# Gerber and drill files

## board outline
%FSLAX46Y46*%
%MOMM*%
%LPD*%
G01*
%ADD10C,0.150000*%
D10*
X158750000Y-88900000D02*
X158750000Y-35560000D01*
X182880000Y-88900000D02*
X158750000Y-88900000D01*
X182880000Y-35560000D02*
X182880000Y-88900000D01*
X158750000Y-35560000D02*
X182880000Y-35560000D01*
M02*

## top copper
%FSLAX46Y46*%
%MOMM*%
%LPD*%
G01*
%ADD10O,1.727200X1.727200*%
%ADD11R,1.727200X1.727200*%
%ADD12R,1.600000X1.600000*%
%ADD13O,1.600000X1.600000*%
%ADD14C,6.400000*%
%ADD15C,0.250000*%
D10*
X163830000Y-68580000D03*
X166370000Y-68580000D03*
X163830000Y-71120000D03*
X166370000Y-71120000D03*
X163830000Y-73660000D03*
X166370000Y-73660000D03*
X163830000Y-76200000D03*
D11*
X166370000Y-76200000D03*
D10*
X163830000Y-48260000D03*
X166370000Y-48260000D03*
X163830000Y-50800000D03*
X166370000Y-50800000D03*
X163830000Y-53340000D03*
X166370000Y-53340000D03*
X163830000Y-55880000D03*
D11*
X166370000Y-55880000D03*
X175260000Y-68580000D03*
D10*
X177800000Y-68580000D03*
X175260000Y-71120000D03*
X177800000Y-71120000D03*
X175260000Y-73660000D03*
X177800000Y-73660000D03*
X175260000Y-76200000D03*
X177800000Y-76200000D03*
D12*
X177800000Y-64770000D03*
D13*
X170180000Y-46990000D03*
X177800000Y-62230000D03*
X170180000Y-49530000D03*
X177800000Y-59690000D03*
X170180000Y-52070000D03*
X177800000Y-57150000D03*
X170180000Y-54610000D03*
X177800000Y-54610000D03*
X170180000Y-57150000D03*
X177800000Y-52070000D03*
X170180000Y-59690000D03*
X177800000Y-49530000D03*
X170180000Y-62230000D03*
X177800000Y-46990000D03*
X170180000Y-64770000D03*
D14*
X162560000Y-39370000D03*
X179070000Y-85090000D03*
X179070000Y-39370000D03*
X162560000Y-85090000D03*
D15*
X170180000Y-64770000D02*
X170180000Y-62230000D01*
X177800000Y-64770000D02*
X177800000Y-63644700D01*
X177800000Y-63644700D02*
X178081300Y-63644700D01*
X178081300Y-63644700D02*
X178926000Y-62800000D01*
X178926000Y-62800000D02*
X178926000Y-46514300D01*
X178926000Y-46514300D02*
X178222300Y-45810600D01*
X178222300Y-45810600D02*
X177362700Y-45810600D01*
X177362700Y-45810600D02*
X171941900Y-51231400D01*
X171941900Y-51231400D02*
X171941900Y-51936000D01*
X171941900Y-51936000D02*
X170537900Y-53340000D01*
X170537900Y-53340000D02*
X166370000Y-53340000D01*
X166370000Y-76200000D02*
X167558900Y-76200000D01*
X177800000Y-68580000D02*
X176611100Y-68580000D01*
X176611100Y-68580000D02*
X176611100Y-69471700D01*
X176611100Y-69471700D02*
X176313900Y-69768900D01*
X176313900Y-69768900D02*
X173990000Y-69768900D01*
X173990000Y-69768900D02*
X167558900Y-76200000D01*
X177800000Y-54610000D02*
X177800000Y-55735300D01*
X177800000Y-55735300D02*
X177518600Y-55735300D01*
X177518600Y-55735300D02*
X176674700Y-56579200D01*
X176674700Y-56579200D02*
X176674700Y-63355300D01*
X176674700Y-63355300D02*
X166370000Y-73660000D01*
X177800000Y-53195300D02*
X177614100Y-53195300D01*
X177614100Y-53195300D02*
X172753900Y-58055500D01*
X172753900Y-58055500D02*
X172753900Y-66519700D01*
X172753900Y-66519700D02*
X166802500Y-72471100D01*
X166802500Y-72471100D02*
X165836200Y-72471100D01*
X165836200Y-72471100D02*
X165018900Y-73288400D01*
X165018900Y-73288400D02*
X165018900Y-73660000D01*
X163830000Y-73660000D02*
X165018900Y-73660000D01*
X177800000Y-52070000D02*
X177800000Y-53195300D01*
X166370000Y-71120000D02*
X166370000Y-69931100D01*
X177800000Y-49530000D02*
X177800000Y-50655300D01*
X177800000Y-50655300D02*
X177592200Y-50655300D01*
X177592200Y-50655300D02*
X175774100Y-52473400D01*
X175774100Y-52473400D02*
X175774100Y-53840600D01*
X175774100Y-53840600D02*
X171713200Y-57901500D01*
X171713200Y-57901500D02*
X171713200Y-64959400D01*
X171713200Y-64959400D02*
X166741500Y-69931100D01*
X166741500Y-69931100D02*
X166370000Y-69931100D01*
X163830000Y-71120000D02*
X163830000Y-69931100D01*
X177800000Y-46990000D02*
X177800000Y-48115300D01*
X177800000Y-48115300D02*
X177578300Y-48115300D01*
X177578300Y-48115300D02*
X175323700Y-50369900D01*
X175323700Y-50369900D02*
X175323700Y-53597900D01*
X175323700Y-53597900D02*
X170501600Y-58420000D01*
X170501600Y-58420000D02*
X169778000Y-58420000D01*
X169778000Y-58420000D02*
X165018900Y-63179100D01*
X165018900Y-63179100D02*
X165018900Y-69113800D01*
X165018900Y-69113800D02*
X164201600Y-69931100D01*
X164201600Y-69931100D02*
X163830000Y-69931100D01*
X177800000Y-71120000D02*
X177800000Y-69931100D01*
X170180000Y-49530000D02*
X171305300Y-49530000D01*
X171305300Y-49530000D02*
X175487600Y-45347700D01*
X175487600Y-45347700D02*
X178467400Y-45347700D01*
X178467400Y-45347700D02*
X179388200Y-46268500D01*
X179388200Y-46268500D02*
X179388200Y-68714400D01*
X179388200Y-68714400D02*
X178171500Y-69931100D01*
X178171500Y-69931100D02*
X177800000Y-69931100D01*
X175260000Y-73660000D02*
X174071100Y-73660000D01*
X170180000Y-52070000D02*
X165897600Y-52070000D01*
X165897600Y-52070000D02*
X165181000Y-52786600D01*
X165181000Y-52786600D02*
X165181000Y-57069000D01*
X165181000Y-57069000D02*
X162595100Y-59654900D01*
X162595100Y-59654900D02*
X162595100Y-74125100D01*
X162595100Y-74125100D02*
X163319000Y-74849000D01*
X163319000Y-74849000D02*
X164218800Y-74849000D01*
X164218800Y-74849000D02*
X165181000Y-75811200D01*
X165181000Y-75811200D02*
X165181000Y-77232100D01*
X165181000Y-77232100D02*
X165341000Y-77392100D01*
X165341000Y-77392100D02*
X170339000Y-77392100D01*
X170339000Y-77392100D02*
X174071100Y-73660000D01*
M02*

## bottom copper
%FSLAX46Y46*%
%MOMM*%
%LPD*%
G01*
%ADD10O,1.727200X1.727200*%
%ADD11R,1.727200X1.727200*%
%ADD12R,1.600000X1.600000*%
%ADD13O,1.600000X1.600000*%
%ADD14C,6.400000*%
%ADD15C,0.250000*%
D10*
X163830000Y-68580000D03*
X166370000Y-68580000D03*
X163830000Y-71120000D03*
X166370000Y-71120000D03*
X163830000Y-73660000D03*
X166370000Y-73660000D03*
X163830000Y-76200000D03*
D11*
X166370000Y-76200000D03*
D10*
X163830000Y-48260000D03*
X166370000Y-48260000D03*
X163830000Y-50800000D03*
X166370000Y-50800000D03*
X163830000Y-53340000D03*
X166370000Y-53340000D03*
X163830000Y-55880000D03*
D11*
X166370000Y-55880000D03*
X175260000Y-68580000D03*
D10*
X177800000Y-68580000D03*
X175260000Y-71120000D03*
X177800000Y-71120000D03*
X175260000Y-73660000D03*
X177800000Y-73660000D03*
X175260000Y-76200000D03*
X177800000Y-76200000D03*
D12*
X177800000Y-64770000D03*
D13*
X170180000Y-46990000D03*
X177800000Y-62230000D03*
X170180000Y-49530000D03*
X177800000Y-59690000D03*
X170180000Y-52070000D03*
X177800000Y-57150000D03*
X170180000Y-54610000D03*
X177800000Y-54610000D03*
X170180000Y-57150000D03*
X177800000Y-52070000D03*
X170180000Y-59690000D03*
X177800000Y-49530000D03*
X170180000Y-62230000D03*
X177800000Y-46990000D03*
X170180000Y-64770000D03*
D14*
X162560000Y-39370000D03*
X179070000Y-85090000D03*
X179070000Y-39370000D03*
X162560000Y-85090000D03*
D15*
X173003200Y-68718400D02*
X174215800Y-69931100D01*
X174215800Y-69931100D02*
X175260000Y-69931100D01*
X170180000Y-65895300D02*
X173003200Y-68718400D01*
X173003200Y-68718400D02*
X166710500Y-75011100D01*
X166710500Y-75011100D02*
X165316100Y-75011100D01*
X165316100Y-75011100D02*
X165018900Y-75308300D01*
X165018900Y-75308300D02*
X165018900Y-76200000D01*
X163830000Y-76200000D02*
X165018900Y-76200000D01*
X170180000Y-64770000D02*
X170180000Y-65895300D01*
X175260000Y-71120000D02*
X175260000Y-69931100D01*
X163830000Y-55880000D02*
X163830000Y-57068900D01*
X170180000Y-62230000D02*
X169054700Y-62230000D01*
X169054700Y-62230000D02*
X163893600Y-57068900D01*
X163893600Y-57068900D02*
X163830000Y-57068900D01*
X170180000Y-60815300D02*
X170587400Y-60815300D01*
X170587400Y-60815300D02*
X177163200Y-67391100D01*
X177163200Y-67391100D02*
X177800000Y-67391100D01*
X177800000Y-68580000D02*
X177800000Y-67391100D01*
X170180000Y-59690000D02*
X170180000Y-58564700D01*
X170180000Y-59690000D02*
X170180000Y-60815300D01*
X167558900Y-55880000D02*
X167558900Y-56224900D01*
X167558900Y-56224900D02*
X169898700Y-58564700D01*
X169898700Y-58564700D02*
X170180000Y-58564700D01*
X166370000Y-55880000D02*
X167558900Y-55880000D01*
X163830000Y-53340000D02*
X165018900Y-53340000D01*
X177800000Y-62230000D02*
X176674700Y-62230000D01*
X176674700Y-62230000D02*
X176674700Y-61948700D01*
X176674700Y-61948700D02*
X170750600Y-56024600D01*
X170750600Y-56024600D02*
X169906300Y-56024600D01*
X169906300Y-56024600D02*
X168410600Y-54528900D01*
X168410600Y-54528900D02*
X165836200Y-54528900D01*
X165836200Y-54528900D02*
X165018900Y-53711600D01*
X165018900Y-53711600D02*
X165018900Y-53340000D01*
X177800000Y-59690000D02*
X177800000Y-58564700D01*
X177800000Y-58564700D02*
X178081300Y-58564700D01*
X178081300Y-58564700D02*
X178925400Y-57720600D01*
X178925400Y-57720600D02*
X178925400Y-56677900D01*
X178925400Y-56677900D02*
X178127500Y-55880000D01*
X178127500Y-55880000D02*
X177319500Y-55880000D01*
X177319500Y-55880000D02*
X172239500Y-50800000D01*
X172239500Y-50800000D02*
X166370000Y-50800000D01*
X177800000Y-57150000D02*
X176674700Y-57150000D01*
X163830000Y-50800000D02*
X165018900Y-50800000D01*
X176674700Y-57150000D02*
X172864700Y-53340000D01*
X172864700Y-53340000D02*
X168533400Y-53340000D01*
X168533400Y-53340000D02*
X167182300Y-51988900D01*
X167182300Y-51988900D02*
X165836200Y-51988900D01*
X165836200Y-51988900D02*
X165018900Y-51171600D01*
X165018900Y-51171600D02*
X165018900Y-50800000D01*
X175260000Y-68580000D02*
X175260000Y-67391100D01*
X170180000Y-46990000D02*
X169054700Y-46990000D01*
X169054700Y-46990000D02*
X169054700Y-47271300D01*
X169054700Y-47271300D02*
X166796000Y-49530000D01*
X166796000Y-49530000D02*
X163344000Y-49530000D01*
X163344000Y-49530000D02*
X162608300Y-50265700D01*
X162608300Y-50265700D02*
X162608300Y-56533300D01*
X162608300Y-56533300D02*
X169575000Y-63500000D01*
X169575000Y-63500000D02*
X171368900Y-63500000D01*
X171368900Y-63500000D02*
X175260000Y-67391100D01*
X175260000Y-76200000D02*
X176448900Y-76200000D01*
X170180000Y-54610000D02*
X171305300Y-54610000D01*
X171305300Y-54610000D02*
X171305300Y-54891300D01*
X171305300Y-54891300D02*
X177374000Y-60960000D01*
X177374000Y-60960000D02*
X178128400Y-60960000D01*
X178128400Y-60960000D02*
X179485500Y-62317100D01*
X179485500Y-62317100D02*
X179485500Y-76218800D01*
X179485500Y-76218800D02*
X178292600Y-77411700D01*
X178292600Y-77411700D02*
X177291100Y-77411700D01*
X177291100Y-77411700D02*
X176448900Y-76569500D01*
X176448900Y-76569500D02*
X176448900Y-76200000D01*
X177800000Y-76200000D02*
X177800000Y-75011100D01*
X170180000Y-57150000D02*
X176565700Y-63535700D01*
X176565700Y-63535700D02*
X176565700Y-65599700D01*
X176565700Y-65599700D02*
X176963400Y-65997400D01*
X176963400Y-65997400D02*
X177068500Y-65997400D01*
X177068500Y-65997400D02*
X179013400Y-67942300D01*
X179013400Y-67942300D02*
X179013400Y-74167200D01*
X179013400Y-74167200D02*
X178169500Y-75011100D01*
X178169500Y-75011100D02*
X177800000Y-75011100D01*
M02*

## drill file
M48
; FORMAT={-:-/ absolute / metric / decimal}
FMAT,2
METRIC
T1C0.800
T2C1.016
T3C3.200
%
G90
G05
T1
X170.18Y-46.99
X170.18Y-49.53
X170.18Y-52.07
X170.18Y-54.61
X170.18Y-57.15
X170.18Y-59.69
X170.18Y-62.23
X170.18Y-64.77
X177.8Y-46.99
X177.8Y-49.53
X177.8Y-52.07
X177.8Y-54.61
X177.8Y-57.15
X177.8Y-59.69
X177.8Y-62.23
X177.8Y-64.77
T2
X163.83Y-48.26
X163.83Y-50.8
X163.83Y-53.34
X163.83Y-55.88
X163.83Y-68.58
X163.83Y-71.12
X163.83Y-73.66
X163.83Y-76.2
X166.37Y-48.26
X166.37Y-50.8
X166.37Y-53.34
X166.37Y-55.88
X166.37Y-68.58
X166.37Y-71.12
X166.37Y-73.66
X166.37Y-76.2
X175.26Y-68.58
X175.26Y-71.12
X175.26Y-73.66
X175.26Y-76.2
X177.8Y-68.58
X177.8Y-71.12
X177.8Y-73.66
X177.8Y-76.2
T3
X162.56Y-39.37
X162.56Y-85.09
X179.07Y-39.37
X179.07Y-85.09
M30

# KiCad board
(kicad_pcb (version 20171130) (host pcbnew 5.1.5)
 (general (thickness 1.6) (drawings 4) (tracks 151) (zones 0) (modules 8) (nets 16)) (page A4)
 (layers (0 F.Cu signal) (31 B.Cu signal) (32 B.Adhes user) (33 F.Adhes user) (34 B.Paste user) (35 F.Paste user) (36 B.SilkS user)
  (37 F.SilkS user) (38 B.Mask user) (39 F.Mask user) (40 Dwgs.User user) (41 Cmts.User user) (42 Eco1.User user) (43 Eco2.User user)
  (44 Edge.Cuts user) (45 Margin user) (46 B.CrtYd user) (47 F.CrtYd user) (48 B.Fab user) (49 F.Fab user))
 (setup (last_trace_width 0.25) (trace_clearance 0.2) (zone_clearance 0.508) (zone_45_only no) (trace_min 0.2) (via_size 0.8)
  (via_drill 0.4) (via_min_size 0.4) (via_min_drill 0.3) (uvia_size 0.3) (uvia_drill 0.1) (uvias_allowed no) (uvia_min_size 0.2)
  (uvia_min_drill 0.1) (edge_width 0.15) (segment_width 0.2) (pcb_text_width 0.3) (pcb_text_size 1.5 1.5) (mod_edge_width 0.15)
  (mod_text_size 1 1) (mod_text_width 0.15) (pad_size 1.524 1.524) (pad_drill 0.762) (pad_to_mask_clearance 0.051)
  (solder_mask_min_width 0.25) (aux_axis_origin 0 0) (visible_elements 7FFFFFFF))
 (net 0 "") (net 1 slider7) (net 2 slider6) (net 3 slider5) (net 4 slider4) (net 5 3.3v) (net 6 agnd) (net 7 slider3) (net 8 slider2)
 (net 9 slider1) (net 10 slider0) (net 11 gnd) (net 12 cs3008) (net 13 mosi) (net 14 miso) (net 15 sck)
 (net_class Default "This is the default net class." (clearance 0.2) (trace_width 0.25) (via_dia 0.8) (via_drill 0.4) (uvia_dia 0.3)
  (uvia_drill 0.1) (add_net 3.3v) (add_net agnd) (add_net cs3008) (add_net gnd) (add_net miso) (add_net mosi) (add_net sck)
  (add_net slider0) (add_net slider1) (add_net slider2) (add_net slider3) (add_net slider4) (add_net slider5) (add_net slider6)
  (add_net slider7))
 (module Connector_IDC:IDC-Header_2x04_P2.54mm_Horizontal (layer F.Cu) (at 166.37 76.2 180)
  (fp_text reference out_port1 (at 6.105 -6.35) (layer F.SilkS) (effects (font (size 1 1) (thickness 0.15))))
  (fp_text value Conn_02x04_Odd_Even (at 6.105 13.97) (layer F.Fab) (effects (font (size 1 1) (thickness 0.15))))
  (pad 8 thru_hole oval (at 2.54 7.62 180) (size 1.7272 1.7272) (drill 1.016) (layers *.Cu *.Mask))
  (pad 7 thru_hole oval (at 0 7.62 180) (size 1.7272 1.7272) (drill 1.016) (layers *.Cu *.Mask))
  (pad 6 thru_hole oval (at 2.54 5.08 180) (size 1.7272 1.7272) (drill 1.016) (layers *.Cu *.Mask) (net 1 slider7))
  (pad 5 thru_hole oval (at 0 5.08 180) (size 1.7272 1.7272) (drill 1.016) (layers *.Cu *.Mask) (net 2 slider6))
  (pad 4 thru_hole oval (at 2.54 2.54 180) (size 1.7272 1.7272) (drill 1.016) (layers *.Cu *.Mask) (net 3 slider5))
  (pad 3 thru_hole oval (at 0 2.54 180) (size 1.7272 1.7272) (drill 1.016) (layers *.Cu *.Mask) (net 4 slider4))
  (pad 2 thru_hole oval (at 2.54 0 180) (size 1.7272 1.7272) (drill 1.016) (layers *.Cu *.Mask) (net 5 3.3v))
  (pad 1 thru_hole rect (at 0 0 180) (size 1.7272 1.7272) (drill 1.016) (layers *.Cu *.Mask) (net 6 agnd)))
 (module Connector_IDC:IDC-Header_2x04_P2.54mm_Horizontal (layer F.Cu) (at 166.37 55.88 180)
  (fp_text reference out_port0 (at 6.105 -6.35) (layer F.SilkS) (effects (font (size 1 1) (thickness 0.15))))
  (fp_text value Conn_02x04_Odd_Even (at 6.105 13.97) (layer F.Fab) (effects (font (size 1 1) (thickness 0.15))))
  (pad 8 thru_hole oval (at 2.54 7.62 180) (size 1.7272 1.7272) (drill 1.016) (layers *.Cu *.Mask))
  (pad 7 thru_hole oval (at 0 7.62 180) (size 1.7272 1.7272) (drill 1.016) (layers *.Cu *.Mask))
  (pad 6 thru_hole oval (at 2.54 5.08 180) (size 1.7272 1.7272) (drill 1.016) (layers *.Cu *.Mask) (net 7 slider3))
  (pad 5 thru_hole oval (at 0 5.08 180) (size 1.7272 1.7272) (drill 1.016) (layers *.Cu *.Mask) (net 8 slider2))
  (pad 4 thru_hole oval (at 2.54 2.54 180) (size 1.7272 1.7272) (drill 1.016) (layers *.Cu *.Mask) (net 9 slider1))
  (pad 3 thru_hole oval (at 0 2.54 180) (size 1.7272 1.7272) (drill 1.016) (layers *.Cu *.Mask) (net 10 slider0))
  (pad 2 thru_hole oval (at 2.54 0 180) (size 1.7272 1.7272) (drill 1.016) (layers *.Cu *.Mask) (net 5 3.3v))
  (pad 1 thru_hole rect (at 0 0 180) (size 1.7272 1.7272) (drill 1.016) (layers *.Cu *.Mask) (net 6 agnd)))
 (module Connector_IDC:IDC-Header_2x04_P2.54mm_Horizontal (layer F.Cu) (at 175.26 68.58)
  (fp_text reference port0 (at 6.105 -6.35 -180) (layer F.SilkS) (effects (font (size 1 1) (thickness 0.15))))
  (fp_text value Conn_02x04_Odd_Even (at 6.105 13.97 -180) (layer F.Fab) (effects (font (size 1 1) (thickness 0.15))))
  (pad 1 thru_hole rect (at 0 0) (size 1.7272 1.7272) (drill 1.016) (layers *.Cu *.Mask) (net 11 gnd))
  (pad 2 thru_hole oval (at 2.54 0) (size 1.7272 1.7272) (drill 1.016) (layers *.Cu *.Mask) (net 6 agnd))
  (pad 3 thru_hole oval (at 0 2.54) (size 1.7272 1.7272) (drill 1.016) (layers *.Cu *.Mask) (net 5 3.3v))
  (pad 4 thru_hole oval (at 2.54 2.54) (size 1.7272 1.7272) (drill 1.016) (layers *.Cu *.Mask) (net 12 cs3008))
  (pad 5 thru_hole oval (at 0 5.08) (size 1.7272 1.7272) (drill 1.016) (layers *.Cu *.Mask) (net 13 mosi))
  (pad 6 thru_hole oval (at 2.54 5.08) (size 1.7272 1.7272) (drill 1.016) (layers *.Cu *.Mask))
  (pad 7 thru_hole oval (at 0 7.62) (size 1.7272 1.7272) (drill 1.016) (layers *.Cu *.Mask) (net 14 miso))
  (pad 8 thru_hole oval (at 2.54 7.62) (size 1.7272 1.7272) (drill 1.016) (layers *.Cu *.Mask) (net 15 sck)))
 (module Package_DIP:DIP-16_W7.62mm (layer F.Cu) (at 177.8 64.77 180)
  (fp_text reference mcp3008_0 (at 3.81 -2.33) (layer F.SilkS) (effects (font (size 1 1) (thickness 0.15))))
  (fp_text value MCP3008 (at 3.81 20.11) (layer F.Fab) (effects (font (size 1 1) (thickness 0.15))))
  (pad 1 thru_hole rect (at 0 0 180) (size 1.6 1.6) (drill 0.8) (layers *.Cu *.Mask) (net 10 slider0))
  (pad 9 thru_hole oval (at 7.62 17.78 180) (size 1.6 1.6) (drill 0.8) (layers *.Cu *.Mask) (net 11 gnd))
  (pad 2 thru_hole oval (at 0 2.54 180) (size 1.6 1.6) (drill 0.8) (layers *.Cu *.Mask) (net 9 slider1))
  (pad 10 thru_hole oval (at 7.62 15.24 180) (size 1.6 1.6) (drill 0.8) (layers *.Cu *.Mask) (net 12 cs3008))
  (pad 3 thru_hole oval (at 0 5.08 180) (size 1.6 1.6) (drill 0.8) (layers *.Cu *.Mask) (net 8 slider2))
  (pad 11 thru_hole oval (at 7.62 12.7 180) (size 1.6 1.6) (drill 0.8) (layers *.Cu *.Mask) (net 13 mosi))
  (pad 4 thru_hole oval (at 0 7.62 180) (size 1.6 1.6) (drill 0.8) (layers *.Cu *.Mask) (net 7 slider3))
  (pad 12 thru_hole oval (at 7.62 10.16 180) (size 1.6 1.6) (drill 0.8) (layers *.Cu *.Mask) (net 14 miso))
  (pad 5 thru_hole oval (at 0 10.16 180) (size 1.6 1.6) (drill 0.8) (layers *.Cu *.Mask) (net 4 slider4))
  (pad 13 thru_hole oval (at 7.62 7.62 180) (size 1.6 1.6) (drill 0.8) (layers *.Cu *.Mask) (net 15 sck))
  (pad 6 thru_hole oval (at 0 12.7 180) (size 1.6 1.6) (drill 0.8) (layers *.Cu *.Mask) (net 3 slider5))
  (pad 14 thru_hole oval (at 7.62 5.08 180) (size 1.6 1.6) (drill 0.8) (layers *.Cu *.Mask) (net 6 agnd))
  (pad 7 thru_hole oval (at 0 15.24 180) (size 1.6 1.6) (drill 0.8) (layers *.Cu *.Mask) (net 2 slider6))
  (pad 15 thru_hole oval (at 7.62 2.54 180) (size 1.6 1.6) (drill 0.8) (layers *.Cu *.Mask) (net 5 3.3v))
  (pad 8 thru_hole oval (at 0 17.78 180) (size 1.6 1.6) (drill 0.8) (layers *.Cu *.Mask) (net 1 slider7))
  (pad 16 thru_hole oval (at 7.62 0 180) (size 1.6 1.6) (drill 0.8) (layers *.Cu *.Mask) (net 5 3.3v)))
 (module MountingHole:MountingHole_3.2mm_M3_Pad (layer F.Cu) (at 162.56 39.37)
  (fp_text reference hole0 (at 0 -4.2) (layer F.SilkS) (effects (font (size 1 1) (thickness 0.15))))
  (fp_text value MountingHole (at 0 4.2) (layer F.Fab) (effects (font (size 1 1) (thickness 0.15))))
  (pad 1 thru_hole circle (at 0 0) (size 6.4 6.4) (drill 3.2) (layers *.Cu *.Mask)))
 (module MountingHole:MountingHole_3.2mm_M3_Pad (layer F.Cu) (at 179.07 85.09)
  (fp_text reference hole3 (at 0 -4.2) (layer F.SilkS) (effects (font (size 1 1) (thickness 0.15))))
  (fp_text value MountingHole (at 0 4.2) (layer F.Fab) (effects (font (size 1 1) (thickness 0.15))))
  (pad 1 thru_hole circle (at 0 0) (size 6.4 6.4) (drill 3.2) (layers *.Cu *.Mask)))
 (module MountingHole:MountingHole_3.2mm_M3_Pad (layer F.Cu) (at 179.07 39.37)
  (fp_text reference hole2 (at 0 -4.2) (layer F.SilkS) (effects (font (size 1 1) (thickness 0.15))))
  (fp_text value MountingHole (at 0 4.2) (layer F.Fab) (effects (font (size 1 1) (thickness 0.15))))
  (pad 1 thru_hole circle (at 0 0) (size 6.4 6.4) (drill 3.2) (layers *.Cu *.Mask)))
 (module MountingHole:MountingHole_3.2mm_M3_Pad (layer F.Cu) (at 162.56 85.09)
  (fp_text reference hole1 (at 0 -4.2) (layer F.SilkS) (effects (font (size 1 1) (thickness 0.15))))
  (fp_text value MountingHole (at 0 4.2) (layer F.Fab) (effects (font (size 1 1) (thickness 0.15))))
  (pad 1 thru_hole circle (at 0 0) (size 6.4 6.4) (drill 3.2) (layers *.Cu *.Mask)))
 (gr_line (start 158.75 88.9) (end 158.75 35.56) (angle 90) (layer Edge.Cuts) (width 0.15))
 (gr_line (start 182.88 88.9) (end 158.75 88.9) (angle 90) (layer Edge.Cuts) (width 0.15))
 (gr_line (start 182.88 35.56) (end 182.88 88.9) (angle 90) (layer Edge.Cuts) (width 0.15))
 (gr_line (start 158.75 35.56) (end 182.88 35.56) (angle 90) (layer Edge.Cuts) (width 0.15))
 (segment (start 173.0032 68.7184) (end 174.2158 69.9311) (width 0.25) (layer B.Cu) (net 5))
 (segment (start 174.2158 69.9311) (end 175.26 69.9311) (width 0.25) (layer B.Cu) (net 5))
 (segment (start 170.18 65.8953) (end 173.0032 68.7184) (width 0.25) (layer B.Cu) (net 5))
 (segment (start 173.0032 68.7184) (end 166.7105 75.0111) (width 0.25) (layer B.Cu) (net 5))
 (segment (start 166.7105 75.0111) (end 165.3161 75.0111) (width 0.25) (layer B.Cu) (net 5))
 (segment (start 165.3161 75.0111) (end 165.0189 75.3083) (width 0.25) (layer B.Cu) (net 5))
 (segment (start 165.0189 75.3083) (end 165.0189 76.2) (width 0.25) (layer B.Cu) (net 5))
 (segment (start 163.83 76.2) (end 165.0189 76.2) (width 0.25) (layer B.Cu) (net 5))
 (segment (start 170.18 64.77) (end 170.18 65.8953) (width 0.25) (layer B.Cu) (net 5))
 (segment (start 175.26 71.12) (end 175.26 69.9311) (width 0.25) (layer B.Cu) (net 5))
 (segment (start 163.83 55.88) (end 163.83 57.0689) (width 0.25) (layer B.Cu) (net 5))
 (segment (start 170.18 62.23) (end 169.0547 62.23) (width 0.25) (layer B.Cu) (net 5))
 (segment (start 169.0547 62.23) (end 163.8936 57.0689) (width 0.25) (layer B.Cu) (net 5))
 (segment (start 163.8936 57.0689) (end 163.83 57.0689) (width 0.25) (layer B.Cu) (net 5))
 (segment (start 170.18 64.77) (end 170.18 62.23) (width 0.25) (layer F.Cu) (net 5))
 (segment (start 177.8 64.77) (end 177.8 63.6447) (width 0.25) (layer F.Cu) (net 10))
 (segment (start 177.8 63.6447) (end 178.0813 63.6447) (width 0.25) (layer F.Cu) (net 10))
 (segment (start 178.0813 63.6447) (end 178.926 62.8) (width 0.25) (layer F.Cu) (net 10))
 (segment (start 178.926 62.8) (end 178.926 46.5143) (width 0.25) (layer F.Cu) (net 10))
 (segment (start 178.926 46.5143) (end 178.2223 45.8106) (width 0.25) (layer F.Cu) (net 10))
 (segment (start 178.2223 45.8106) (end 177.3627 45.8106) (width 0.25) (layer F.Cu) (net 10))
 (segment (start 177.3627 45.8106) (end 171.9419 51.2314) (width 0.25) (layer F.Cu) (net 10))
 (segment (start 171.9419 51.2314) (end 171.9419 51.936) (width 0.25) (layer F.Cu) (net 10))
 (segment (start 171.9419 51.936) (end 170.5379 53.34) (width 0.25) (layer F.Cu) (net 10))
 (segment (start 170.5379 53.34) (end 166.37 53.34) (width 0.25) (layer F.Cu) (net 10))
 (segment (start 170.18 60.8153) (end 170.5874 60.8153) (width 0.25) (layer B.Cu) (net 6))
 (segment (start 170.5874 60.8153) (end 177.1632 67.3911) (width 0.25) (layer B.Cu) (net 6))
 (segment (start 177.1632 67.3911) (end 177.8 67.3911) (width 0.25) (layer B.Cu) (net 6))
 (segment (start 166.37 76.2) (end 167.5589 76.2) (width 0.25) (layer F.Cu) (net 6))
 (segment (start 177.8 68.58) (end 176.6111 68.58) (width 0.25) (layer F.Cu) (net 6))
 (segment (start 176.6111 68.58) (end 176.6111 69.4717) (width 0.25) (layer F.Cu) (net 6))
 (segment (start 176.6111 69.4717) (end 176.3139 69.7689) (width 0.25) (layer F.Cu) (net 6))
 (segment (start 176.3139 69.7689) (end 173.99 69.7689) (width 0.25) (layer F.Cu) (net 6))
 (segment (start 173.99 69.7689) (end 167.5589 76.2) (width 0.25) (layer F.Cu) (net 6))
 (segment (start 177.8 68.58) (end 177.8 67.3911) (width 0.25) (layer B.Cu) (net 6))
 (segment (start 170.18 59.69) (end 170.18 58.5647) (width 0.25) (layer B.Cu) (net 6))
 (segment (start 170.18 59.69) (end 170.18 60.8153) (width 0.25) (layer B.Cu) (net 6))
 (segment (start 167.5589 55.88) (end 167.5589 56.2249) (width 0.25) (layer B.Cu) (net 6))
 (segment (start 167.5589 56.2249) (end 169.8987 58.5647) (width 0.25) (layer B.Cu) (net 6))
 (segment (start 169.8987 58.5647) (end 170.18 58.5647) (width 0.25) (layer B.Cu) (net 6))
 (segment (start 166.37 55.88) (end 167.5589 55.88) (width 0.25) (layer B.Cu) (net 6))
 (segment (start 177.8 54.61) (end 177.8 55.7353) (width 0.25) (layer F.Cu) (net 4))
 (segment (start 177.8 55.7353) (end 177.5186 55.7353) (width 0.25) (layer F.Cu) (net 4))
 (segment (start 177.5186 55.7353) (end 176.6747 56.5792) (width 0.25) (layer F.Cu) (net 4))
 (segment (start 176.6747 56.5792) (end 176.6747 63.3553) (width 0.25) (layer F.Cu) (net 4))
 (segment (start 176.6747 63.3553) (end 166.37 73.66) (width 0.25) (layer F.Cu) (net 4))
 (segment (start 163.83 53.34) (end 165.0189 53.34) (width 0.25) (layer B.Cu) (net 9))
 (segment (start 177.8 62.23) (end 176.6747 62.23) (width 0.25) (layer B.Cu) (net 9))
 (segment (start 176.6747 62.23) (end 176.6747 61.9487) (width 0.25) (layer B.Cu) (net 9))
 (segment (start 176.6747 61.9487) (end 170.7506 56.0246) (width 0.25) (layer B.Cu) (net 9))
 (segment (start 170.7506 56.0246) (end 169.9063 56.0246) (width 0.25) (layer B.Cu) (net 9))
 (segment (start 169.9063 56.0246) (end 168.4106 54.5289) (width 0.25) (layer B.Cu) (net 9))
 (segment (start 168.4106 54.5289) (end 165.8362 54.5289) (width 0.25) (layer B.Cu) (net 9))
 (segment (start 165.8362 54.5289) (end 165.0189 53.7116) (width 0.25) (layer B.Cu) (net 9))
 (segment (start 165.0189 53.7116) (end 165.0189 53.34) (width 0.25) (layer B.Cu) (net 9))
 (segment (start 177.8 53.1953) (end 177.6141 53.1953) (width 0.25) (layer F.Cu) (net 3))
 (segment (start 177.6141 53.1953) (end 172.7539 58.0555) (width 0.25) (layer F.Cu) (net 3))
 (segment (start 172.7539 58.0555) (end 172.7539 66.5197) (width 0.25) (layer F.Cu) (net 3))
 (segment (start 172.7539 66.5197) (end 166.8025 72.4711) (width 0.25) (layer F.Cu) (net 3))
 (segment (start 166.8025 72.4711) (end 165.8362 72.4711) (width 0.25) (layer F.Cu) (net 3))
 (segment (start 165.8362 72.4711) (end 165.0189 73.2884) (width 0.25) (layer F.Cu) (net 3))
 (segment (start 165.0189 73.2884) (end 165.0189 73.66) (width 0.25) (layer F.Cu) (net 3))
 (segment (start 163.83 73.66) (end 165.0189 73.66) (width 0.25) (layer F.Cu) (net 3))
 (segment (start 177.8 52.07) (end 177.8 53.1953) (width 0.25) (layer F.Cu) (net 3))
 (segment (start 177.8 59.69) (end 177.8 58.5647) (width 0.25) (layer B.Cu) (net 8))
 (segment (start 177.8 58.5647) (end 178.0813 58.5647) (width 0.25) (layer B.Cu) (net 8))
 (segment (start 178.0813 58.5647) (end 178.9254 57.7206) (width 0.25) (layer B.Cu) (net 8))
 (segment (start 178.9254 57.7206) (end 178.9254 56.6779) (width 0.25) (layer B.Cu) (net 8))
 (segment (start 178.9254 56.6779) (end 178.1275 55.88) (width 0.25) (layer B.Cu) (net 8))
 (segment (start 178.1275 55.88) (end 177.3195 55.88) (width 0.25) (layer B.Cu) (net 8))
 (segment (start 177.3195 55.88) (end 172.2395 50.8) (width 0.25) (layer B.Cu) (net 8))
 (segment (start 172.2395 50.8) (end 166.37 50.8) (width 0.25) (layer B.Cu) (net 8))
 (segment (start 166.37 71.12) (end 166.37 69.9311) (width 0.25) (layer F.Cu) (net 2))
 (segment (start 177.8 49.53) (end 177.8 50.6553) (width 0.25) (layer F.Cu) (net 2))
 (segment (start 177.8 50.6553) (end 177.5922 50.6553) (width 0.25) (layer F.Cu) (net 2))
 (segment (start 177.5922 50.6553) (end 175.7741 52.4734) (width 0.25) (layer F.Cu) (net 2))
 (segment (start 175.7741 52.4734) (end 175.7741 53.8406) (width 0.25) (layer F.Cu) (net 2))
 (segment (start 175.7741 53.8406) (end 171.7132 57.9015) (width 0.25) (layer F.Cu) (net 2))
 (segment (start 171.7132 57.9015) (end 171.7132 64.9594) (width 0.25) (layer F.Cu) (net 2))
 (segment (start 171.7132 64.9594) (end 166.7415 69.9311) (width 0.25) (layer F.Cu) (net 2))
 (segment (start 166.7415 69.9311) (end 166.37 69.9311) (width 0.25) (layer F.Cu) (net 2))
 (segment (start 177.8 57.15) (end 176.6747 57.15) (width 0.25) (layer B.Cu) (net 7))
 (segment (start 163.83 50.8) (end 165.0189 50.8) (width 0.25) (layer B.Cu) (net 7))
 (segment (start 176.6747 57.15) (end 172.8647 53.34) (width 0.25) (layer B.Cu) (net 7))
 (segment (start 172.8647 53.34) (end 168.5334 53.34) (width 0.25) (layer B.Cu) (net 7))
 (segment (start 168.5334 53.34) (end 167.1823 51.9889) (width 0.25) (layer B.Cu) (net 7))
 (segment (start 167.1823 51.9889) (end 165.8362 51.9889) (width 0.25) (layer B.Cu) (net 7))
 (segment (start 165.8362 51.9889) (end 165.0189 51.1716) (width 0.25) (layer B.Cu) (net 7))
 (segment (start 165.0189 51.1716) (end 165.0189 50.8) (width 0.25) (layer B.Cu) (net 7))
 (segment (start 163.83 71.12) (end 163.83 69.9311) (width 0.25) (layer F.Cu) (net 1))
 (segment (start 177.8 46.99) (end 177.8 48.1153) (width 0.25) (layer F.Cu) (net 1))
 (segment (start 177.8 48.1153) (end 177.5783 48.1153) (width 0.25) (layer F.Cu) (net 1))
 (segment (start 177.5783 48.1153) (end 175.3237 50.3699) (width 0.25) (layer F.Cu) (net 1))
 (segment (start 175.3237 50.3699) (end 175.3237 53.5979) (width 0.25) (layer F.Cu) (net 1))
 (segment (start 175.3237 53.5979) (end 170.5016 58.42) (width 0.25) (layer F.Cu) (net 1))
 (segment (start 170.5016 58.42) (end 169.778 58.42) (width 0.25) (layer F.Cu) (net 1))
 (segment (start 169.778 58.42) (end 165.0189 63.1791) (width 0.25) (layer F.Cu) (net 1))
 (segment (start 165.0189 63.1791) (end 165.0189 69.1138) (width 0.25) (layer F.Cu) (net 1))
 (segment (start 165.0189 69.1138) (end 164.2016 69.9311) (width 0.25) (layer F.Cu) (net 1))
 (segment (start 164.2016 69.9311) (end 163.83 69.9311) (width 0.25) (layer F.Cu) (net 1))
 (segment (start 175.26 68.58) (end 175.26 67.3911) (width 0.25) (layer B.Cu) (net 11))
 (segment (start 170.18 46.99) (end 169.0547 46.99) (width 0.25) (layer B.Cu) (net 11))
 (segment (start 169.0547 46.99) (end 169.0547 47.2713) (width 0.25) (layer B.Cu) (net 11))
 (segment (start 169.0547 47.2713) (end 166.796 49.53) (width 0.25) (layer B.Cu) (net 11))
 (segment (start 166.796 49.53) (end 163.344 49.53) (width 0.25) (layer B.Cu) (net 11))
 (segment (start 163.344 49.53) (end 162.6083 50.2657) (width 0.25) (layer B.Cu) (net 11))
 (segment (start 162.6083 50.2657) (end 162.6083 56.5333) (width 0.25) (layer B.Cu) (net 11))
 (segment (start 162.6083 56.5333) (end 169.575 63.5) (width 0.25) (layer B.Cu) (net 11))
 (segment (start 169.575 63.5) (end 171.3689 63.5) (width 0.25) (layer B.Cu) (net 11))
 (segment (start 171.3689 63.5) (end 175.26 67.3911) (width 0.25) (layer B.Cu) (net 11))
 (segment (start 177.8 71.12) (end 177.8 69.9311) (width 0.25) (layer F.Cu) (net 12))
 (segment (start 170.18 49.53) (end 171.3053 49.53) (width 0.25) (layer F.Cu) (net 12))
 (segment (start 171.3053 49.53) (end 175.4876 45.3477) (width 0.25) (layer F.Cu) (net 12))
 (segment (start 175.4876 45.3477) (end 178.4674 45.3477) (width 0.25) (layer F.Cu) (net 12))
 (segment (start 178.4674 45.3477) (end 179.3882 46.2685) (width 0.25) (layer F.Cu) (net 12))
 (segment (start 179.3882 46.2685) (end 179.3882 68.7144) (width 0.25) (layer F.Cu) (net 12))
 (segment (start 179.3882 68.7144) (end 178.1715 69.9311) (width 0.25) (layer F.Cu) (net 12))
 (segment (start 178.1715 69.9311) (end 177.8 69.9311) (width 0.25) (layer F.Cu) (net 12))
 (segment (start 175.26 73.66) (end 174.0711 73.66) (width 0.25) (layer F.Cu) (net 13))
 (segment (start 170.18 52.07) (end 165.8976 52.07) (width 0.25) (layer F.Cu) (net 13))
 (segment (start 165.8976 52.07) (end 165.181 52.7866) (width 0.25) (layer F.Cu) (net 13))
 (segment (start 165.181 52.7866) (end 165.181 57.069) (width 0.25) (layer F.Cu) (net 13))
 (segment (start 165.181 57.069) (end 162.5951 59.6549) (width 0.25) (layer F.Cu) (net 13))
 (segment (start 162.5951 59.6549) (end 162.5951 74.1251) (width 0.25) (layer F.Cu) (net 13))
 (segment (start 162.5951 74.1251) (end 163.319 74.849) (width 0.25) (layer F.Cu) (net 13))
 (segment (start 163.319 74.849) (end 164.2188 74.849) (width 0.25) (layer F.Cu) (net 13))
 (segment (start 164.2188 74.849) (end 165.181 75.8112) (width 0.25) (layer F.Cu) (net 13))
 (segment (start 165.181 75.8112) (end 165.181 77.2321) (width 0.25) (layer F.Cu) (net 13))
 (segment (start 165.181 77.2321) (end 165.341 77.3921) (width 0.25) (layer F.Cu) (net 13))
 (segment (start 165.341 77.3921) (end 170.339 77.3921) (width 0.25) (layer F.Cu) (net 13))
 (segment (start 170.339 77.3921) (end 174.0711 73.66) (width 0.25) (layer F.Cu) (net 13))
 (segment (start 175.26 76.2) (end 176.4489 76.2) (width 0.25) (layer B.Cu) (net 14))
 (segment (start 170.18 54.61) (end 171.3053 54.61) (width 0.25) (layer B.Cu) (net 14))
 (segment (start 171.3053 54.61) (end 171.3053 54.8913) (width 0.25) (layer B.Cu) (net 14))
 (segment (start 171.3053 54.8913) (end 177.374 60.96) (width 0.25) (layer B.Cu) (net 14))
 (segment (start 177.374 60.96) (end 178.1284 60.96) (width 0.25) (layer B.Cu) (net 14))
 (segment (start 178.1284 60.96) (end 179.4855 62.3171) (width 0.25) (layer B.Cu) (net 14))
 (segment (start 179.4855 62.3171) (end 179.4855 76.2188) (width 0.25) (layer B.Cu) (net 14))
 (segment (start 179.4855 76.2188) (end 178.2926 77.4117) (width 0.25) (layer B.Cu) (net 14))
 (segment (start 178.2926 77.4117) (end 177.2911 77.4117) (width 0.25) (layer B.Cu) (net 14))
 (segment (start 177.2911 77.4117) (end 176.4489 76.5695) (width 0.25) (layer B.Cu) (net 14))
 (segment (start 176.4489 76.5695) (end 176.4489 76.2) (width 0.25) (layer B.Cu) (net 14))
 (segment (start 177.8 76.2) (end 177.8 75.0111) (width 0.25) (layer B.Cu) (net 15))
 (segment (start 170.18 57.15) (end 176.5657 63.5357) (width 0.25) (layer B.Cu) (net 15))
 (segment (start 176.5657 63.5357) (end 176.5657 65.5997) (width 0.25) (layer B.Cu) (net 15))
 (segment (start 176.5657 65.5997) (end 176.9634 65.9974) (width 0.25) (layer B.Cu) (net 15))
 (segment (start 176.9634 65.9974) (end 177.0685 65.9974) (width 0.25) (layer B.Cu) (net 15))
 (segment (start 177.0685 65.9974) (end 179.0134 67.9423) (width 0.25) (layer B.Cu) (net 15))
 (segment (start 179.0134 67.9423) (end 179.0134 74.1672) (width 0.25) (layer B.Cu) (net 15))
 (segment (start 179.0134 74.1672) (end 178.1695 75.0111) (width 0.25) (layer B.Cu) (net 15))
 (segment (start 178.1695 75.0111) (end 177.8 75.0111) (width 0.25) (layer B.Cu) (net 15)))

